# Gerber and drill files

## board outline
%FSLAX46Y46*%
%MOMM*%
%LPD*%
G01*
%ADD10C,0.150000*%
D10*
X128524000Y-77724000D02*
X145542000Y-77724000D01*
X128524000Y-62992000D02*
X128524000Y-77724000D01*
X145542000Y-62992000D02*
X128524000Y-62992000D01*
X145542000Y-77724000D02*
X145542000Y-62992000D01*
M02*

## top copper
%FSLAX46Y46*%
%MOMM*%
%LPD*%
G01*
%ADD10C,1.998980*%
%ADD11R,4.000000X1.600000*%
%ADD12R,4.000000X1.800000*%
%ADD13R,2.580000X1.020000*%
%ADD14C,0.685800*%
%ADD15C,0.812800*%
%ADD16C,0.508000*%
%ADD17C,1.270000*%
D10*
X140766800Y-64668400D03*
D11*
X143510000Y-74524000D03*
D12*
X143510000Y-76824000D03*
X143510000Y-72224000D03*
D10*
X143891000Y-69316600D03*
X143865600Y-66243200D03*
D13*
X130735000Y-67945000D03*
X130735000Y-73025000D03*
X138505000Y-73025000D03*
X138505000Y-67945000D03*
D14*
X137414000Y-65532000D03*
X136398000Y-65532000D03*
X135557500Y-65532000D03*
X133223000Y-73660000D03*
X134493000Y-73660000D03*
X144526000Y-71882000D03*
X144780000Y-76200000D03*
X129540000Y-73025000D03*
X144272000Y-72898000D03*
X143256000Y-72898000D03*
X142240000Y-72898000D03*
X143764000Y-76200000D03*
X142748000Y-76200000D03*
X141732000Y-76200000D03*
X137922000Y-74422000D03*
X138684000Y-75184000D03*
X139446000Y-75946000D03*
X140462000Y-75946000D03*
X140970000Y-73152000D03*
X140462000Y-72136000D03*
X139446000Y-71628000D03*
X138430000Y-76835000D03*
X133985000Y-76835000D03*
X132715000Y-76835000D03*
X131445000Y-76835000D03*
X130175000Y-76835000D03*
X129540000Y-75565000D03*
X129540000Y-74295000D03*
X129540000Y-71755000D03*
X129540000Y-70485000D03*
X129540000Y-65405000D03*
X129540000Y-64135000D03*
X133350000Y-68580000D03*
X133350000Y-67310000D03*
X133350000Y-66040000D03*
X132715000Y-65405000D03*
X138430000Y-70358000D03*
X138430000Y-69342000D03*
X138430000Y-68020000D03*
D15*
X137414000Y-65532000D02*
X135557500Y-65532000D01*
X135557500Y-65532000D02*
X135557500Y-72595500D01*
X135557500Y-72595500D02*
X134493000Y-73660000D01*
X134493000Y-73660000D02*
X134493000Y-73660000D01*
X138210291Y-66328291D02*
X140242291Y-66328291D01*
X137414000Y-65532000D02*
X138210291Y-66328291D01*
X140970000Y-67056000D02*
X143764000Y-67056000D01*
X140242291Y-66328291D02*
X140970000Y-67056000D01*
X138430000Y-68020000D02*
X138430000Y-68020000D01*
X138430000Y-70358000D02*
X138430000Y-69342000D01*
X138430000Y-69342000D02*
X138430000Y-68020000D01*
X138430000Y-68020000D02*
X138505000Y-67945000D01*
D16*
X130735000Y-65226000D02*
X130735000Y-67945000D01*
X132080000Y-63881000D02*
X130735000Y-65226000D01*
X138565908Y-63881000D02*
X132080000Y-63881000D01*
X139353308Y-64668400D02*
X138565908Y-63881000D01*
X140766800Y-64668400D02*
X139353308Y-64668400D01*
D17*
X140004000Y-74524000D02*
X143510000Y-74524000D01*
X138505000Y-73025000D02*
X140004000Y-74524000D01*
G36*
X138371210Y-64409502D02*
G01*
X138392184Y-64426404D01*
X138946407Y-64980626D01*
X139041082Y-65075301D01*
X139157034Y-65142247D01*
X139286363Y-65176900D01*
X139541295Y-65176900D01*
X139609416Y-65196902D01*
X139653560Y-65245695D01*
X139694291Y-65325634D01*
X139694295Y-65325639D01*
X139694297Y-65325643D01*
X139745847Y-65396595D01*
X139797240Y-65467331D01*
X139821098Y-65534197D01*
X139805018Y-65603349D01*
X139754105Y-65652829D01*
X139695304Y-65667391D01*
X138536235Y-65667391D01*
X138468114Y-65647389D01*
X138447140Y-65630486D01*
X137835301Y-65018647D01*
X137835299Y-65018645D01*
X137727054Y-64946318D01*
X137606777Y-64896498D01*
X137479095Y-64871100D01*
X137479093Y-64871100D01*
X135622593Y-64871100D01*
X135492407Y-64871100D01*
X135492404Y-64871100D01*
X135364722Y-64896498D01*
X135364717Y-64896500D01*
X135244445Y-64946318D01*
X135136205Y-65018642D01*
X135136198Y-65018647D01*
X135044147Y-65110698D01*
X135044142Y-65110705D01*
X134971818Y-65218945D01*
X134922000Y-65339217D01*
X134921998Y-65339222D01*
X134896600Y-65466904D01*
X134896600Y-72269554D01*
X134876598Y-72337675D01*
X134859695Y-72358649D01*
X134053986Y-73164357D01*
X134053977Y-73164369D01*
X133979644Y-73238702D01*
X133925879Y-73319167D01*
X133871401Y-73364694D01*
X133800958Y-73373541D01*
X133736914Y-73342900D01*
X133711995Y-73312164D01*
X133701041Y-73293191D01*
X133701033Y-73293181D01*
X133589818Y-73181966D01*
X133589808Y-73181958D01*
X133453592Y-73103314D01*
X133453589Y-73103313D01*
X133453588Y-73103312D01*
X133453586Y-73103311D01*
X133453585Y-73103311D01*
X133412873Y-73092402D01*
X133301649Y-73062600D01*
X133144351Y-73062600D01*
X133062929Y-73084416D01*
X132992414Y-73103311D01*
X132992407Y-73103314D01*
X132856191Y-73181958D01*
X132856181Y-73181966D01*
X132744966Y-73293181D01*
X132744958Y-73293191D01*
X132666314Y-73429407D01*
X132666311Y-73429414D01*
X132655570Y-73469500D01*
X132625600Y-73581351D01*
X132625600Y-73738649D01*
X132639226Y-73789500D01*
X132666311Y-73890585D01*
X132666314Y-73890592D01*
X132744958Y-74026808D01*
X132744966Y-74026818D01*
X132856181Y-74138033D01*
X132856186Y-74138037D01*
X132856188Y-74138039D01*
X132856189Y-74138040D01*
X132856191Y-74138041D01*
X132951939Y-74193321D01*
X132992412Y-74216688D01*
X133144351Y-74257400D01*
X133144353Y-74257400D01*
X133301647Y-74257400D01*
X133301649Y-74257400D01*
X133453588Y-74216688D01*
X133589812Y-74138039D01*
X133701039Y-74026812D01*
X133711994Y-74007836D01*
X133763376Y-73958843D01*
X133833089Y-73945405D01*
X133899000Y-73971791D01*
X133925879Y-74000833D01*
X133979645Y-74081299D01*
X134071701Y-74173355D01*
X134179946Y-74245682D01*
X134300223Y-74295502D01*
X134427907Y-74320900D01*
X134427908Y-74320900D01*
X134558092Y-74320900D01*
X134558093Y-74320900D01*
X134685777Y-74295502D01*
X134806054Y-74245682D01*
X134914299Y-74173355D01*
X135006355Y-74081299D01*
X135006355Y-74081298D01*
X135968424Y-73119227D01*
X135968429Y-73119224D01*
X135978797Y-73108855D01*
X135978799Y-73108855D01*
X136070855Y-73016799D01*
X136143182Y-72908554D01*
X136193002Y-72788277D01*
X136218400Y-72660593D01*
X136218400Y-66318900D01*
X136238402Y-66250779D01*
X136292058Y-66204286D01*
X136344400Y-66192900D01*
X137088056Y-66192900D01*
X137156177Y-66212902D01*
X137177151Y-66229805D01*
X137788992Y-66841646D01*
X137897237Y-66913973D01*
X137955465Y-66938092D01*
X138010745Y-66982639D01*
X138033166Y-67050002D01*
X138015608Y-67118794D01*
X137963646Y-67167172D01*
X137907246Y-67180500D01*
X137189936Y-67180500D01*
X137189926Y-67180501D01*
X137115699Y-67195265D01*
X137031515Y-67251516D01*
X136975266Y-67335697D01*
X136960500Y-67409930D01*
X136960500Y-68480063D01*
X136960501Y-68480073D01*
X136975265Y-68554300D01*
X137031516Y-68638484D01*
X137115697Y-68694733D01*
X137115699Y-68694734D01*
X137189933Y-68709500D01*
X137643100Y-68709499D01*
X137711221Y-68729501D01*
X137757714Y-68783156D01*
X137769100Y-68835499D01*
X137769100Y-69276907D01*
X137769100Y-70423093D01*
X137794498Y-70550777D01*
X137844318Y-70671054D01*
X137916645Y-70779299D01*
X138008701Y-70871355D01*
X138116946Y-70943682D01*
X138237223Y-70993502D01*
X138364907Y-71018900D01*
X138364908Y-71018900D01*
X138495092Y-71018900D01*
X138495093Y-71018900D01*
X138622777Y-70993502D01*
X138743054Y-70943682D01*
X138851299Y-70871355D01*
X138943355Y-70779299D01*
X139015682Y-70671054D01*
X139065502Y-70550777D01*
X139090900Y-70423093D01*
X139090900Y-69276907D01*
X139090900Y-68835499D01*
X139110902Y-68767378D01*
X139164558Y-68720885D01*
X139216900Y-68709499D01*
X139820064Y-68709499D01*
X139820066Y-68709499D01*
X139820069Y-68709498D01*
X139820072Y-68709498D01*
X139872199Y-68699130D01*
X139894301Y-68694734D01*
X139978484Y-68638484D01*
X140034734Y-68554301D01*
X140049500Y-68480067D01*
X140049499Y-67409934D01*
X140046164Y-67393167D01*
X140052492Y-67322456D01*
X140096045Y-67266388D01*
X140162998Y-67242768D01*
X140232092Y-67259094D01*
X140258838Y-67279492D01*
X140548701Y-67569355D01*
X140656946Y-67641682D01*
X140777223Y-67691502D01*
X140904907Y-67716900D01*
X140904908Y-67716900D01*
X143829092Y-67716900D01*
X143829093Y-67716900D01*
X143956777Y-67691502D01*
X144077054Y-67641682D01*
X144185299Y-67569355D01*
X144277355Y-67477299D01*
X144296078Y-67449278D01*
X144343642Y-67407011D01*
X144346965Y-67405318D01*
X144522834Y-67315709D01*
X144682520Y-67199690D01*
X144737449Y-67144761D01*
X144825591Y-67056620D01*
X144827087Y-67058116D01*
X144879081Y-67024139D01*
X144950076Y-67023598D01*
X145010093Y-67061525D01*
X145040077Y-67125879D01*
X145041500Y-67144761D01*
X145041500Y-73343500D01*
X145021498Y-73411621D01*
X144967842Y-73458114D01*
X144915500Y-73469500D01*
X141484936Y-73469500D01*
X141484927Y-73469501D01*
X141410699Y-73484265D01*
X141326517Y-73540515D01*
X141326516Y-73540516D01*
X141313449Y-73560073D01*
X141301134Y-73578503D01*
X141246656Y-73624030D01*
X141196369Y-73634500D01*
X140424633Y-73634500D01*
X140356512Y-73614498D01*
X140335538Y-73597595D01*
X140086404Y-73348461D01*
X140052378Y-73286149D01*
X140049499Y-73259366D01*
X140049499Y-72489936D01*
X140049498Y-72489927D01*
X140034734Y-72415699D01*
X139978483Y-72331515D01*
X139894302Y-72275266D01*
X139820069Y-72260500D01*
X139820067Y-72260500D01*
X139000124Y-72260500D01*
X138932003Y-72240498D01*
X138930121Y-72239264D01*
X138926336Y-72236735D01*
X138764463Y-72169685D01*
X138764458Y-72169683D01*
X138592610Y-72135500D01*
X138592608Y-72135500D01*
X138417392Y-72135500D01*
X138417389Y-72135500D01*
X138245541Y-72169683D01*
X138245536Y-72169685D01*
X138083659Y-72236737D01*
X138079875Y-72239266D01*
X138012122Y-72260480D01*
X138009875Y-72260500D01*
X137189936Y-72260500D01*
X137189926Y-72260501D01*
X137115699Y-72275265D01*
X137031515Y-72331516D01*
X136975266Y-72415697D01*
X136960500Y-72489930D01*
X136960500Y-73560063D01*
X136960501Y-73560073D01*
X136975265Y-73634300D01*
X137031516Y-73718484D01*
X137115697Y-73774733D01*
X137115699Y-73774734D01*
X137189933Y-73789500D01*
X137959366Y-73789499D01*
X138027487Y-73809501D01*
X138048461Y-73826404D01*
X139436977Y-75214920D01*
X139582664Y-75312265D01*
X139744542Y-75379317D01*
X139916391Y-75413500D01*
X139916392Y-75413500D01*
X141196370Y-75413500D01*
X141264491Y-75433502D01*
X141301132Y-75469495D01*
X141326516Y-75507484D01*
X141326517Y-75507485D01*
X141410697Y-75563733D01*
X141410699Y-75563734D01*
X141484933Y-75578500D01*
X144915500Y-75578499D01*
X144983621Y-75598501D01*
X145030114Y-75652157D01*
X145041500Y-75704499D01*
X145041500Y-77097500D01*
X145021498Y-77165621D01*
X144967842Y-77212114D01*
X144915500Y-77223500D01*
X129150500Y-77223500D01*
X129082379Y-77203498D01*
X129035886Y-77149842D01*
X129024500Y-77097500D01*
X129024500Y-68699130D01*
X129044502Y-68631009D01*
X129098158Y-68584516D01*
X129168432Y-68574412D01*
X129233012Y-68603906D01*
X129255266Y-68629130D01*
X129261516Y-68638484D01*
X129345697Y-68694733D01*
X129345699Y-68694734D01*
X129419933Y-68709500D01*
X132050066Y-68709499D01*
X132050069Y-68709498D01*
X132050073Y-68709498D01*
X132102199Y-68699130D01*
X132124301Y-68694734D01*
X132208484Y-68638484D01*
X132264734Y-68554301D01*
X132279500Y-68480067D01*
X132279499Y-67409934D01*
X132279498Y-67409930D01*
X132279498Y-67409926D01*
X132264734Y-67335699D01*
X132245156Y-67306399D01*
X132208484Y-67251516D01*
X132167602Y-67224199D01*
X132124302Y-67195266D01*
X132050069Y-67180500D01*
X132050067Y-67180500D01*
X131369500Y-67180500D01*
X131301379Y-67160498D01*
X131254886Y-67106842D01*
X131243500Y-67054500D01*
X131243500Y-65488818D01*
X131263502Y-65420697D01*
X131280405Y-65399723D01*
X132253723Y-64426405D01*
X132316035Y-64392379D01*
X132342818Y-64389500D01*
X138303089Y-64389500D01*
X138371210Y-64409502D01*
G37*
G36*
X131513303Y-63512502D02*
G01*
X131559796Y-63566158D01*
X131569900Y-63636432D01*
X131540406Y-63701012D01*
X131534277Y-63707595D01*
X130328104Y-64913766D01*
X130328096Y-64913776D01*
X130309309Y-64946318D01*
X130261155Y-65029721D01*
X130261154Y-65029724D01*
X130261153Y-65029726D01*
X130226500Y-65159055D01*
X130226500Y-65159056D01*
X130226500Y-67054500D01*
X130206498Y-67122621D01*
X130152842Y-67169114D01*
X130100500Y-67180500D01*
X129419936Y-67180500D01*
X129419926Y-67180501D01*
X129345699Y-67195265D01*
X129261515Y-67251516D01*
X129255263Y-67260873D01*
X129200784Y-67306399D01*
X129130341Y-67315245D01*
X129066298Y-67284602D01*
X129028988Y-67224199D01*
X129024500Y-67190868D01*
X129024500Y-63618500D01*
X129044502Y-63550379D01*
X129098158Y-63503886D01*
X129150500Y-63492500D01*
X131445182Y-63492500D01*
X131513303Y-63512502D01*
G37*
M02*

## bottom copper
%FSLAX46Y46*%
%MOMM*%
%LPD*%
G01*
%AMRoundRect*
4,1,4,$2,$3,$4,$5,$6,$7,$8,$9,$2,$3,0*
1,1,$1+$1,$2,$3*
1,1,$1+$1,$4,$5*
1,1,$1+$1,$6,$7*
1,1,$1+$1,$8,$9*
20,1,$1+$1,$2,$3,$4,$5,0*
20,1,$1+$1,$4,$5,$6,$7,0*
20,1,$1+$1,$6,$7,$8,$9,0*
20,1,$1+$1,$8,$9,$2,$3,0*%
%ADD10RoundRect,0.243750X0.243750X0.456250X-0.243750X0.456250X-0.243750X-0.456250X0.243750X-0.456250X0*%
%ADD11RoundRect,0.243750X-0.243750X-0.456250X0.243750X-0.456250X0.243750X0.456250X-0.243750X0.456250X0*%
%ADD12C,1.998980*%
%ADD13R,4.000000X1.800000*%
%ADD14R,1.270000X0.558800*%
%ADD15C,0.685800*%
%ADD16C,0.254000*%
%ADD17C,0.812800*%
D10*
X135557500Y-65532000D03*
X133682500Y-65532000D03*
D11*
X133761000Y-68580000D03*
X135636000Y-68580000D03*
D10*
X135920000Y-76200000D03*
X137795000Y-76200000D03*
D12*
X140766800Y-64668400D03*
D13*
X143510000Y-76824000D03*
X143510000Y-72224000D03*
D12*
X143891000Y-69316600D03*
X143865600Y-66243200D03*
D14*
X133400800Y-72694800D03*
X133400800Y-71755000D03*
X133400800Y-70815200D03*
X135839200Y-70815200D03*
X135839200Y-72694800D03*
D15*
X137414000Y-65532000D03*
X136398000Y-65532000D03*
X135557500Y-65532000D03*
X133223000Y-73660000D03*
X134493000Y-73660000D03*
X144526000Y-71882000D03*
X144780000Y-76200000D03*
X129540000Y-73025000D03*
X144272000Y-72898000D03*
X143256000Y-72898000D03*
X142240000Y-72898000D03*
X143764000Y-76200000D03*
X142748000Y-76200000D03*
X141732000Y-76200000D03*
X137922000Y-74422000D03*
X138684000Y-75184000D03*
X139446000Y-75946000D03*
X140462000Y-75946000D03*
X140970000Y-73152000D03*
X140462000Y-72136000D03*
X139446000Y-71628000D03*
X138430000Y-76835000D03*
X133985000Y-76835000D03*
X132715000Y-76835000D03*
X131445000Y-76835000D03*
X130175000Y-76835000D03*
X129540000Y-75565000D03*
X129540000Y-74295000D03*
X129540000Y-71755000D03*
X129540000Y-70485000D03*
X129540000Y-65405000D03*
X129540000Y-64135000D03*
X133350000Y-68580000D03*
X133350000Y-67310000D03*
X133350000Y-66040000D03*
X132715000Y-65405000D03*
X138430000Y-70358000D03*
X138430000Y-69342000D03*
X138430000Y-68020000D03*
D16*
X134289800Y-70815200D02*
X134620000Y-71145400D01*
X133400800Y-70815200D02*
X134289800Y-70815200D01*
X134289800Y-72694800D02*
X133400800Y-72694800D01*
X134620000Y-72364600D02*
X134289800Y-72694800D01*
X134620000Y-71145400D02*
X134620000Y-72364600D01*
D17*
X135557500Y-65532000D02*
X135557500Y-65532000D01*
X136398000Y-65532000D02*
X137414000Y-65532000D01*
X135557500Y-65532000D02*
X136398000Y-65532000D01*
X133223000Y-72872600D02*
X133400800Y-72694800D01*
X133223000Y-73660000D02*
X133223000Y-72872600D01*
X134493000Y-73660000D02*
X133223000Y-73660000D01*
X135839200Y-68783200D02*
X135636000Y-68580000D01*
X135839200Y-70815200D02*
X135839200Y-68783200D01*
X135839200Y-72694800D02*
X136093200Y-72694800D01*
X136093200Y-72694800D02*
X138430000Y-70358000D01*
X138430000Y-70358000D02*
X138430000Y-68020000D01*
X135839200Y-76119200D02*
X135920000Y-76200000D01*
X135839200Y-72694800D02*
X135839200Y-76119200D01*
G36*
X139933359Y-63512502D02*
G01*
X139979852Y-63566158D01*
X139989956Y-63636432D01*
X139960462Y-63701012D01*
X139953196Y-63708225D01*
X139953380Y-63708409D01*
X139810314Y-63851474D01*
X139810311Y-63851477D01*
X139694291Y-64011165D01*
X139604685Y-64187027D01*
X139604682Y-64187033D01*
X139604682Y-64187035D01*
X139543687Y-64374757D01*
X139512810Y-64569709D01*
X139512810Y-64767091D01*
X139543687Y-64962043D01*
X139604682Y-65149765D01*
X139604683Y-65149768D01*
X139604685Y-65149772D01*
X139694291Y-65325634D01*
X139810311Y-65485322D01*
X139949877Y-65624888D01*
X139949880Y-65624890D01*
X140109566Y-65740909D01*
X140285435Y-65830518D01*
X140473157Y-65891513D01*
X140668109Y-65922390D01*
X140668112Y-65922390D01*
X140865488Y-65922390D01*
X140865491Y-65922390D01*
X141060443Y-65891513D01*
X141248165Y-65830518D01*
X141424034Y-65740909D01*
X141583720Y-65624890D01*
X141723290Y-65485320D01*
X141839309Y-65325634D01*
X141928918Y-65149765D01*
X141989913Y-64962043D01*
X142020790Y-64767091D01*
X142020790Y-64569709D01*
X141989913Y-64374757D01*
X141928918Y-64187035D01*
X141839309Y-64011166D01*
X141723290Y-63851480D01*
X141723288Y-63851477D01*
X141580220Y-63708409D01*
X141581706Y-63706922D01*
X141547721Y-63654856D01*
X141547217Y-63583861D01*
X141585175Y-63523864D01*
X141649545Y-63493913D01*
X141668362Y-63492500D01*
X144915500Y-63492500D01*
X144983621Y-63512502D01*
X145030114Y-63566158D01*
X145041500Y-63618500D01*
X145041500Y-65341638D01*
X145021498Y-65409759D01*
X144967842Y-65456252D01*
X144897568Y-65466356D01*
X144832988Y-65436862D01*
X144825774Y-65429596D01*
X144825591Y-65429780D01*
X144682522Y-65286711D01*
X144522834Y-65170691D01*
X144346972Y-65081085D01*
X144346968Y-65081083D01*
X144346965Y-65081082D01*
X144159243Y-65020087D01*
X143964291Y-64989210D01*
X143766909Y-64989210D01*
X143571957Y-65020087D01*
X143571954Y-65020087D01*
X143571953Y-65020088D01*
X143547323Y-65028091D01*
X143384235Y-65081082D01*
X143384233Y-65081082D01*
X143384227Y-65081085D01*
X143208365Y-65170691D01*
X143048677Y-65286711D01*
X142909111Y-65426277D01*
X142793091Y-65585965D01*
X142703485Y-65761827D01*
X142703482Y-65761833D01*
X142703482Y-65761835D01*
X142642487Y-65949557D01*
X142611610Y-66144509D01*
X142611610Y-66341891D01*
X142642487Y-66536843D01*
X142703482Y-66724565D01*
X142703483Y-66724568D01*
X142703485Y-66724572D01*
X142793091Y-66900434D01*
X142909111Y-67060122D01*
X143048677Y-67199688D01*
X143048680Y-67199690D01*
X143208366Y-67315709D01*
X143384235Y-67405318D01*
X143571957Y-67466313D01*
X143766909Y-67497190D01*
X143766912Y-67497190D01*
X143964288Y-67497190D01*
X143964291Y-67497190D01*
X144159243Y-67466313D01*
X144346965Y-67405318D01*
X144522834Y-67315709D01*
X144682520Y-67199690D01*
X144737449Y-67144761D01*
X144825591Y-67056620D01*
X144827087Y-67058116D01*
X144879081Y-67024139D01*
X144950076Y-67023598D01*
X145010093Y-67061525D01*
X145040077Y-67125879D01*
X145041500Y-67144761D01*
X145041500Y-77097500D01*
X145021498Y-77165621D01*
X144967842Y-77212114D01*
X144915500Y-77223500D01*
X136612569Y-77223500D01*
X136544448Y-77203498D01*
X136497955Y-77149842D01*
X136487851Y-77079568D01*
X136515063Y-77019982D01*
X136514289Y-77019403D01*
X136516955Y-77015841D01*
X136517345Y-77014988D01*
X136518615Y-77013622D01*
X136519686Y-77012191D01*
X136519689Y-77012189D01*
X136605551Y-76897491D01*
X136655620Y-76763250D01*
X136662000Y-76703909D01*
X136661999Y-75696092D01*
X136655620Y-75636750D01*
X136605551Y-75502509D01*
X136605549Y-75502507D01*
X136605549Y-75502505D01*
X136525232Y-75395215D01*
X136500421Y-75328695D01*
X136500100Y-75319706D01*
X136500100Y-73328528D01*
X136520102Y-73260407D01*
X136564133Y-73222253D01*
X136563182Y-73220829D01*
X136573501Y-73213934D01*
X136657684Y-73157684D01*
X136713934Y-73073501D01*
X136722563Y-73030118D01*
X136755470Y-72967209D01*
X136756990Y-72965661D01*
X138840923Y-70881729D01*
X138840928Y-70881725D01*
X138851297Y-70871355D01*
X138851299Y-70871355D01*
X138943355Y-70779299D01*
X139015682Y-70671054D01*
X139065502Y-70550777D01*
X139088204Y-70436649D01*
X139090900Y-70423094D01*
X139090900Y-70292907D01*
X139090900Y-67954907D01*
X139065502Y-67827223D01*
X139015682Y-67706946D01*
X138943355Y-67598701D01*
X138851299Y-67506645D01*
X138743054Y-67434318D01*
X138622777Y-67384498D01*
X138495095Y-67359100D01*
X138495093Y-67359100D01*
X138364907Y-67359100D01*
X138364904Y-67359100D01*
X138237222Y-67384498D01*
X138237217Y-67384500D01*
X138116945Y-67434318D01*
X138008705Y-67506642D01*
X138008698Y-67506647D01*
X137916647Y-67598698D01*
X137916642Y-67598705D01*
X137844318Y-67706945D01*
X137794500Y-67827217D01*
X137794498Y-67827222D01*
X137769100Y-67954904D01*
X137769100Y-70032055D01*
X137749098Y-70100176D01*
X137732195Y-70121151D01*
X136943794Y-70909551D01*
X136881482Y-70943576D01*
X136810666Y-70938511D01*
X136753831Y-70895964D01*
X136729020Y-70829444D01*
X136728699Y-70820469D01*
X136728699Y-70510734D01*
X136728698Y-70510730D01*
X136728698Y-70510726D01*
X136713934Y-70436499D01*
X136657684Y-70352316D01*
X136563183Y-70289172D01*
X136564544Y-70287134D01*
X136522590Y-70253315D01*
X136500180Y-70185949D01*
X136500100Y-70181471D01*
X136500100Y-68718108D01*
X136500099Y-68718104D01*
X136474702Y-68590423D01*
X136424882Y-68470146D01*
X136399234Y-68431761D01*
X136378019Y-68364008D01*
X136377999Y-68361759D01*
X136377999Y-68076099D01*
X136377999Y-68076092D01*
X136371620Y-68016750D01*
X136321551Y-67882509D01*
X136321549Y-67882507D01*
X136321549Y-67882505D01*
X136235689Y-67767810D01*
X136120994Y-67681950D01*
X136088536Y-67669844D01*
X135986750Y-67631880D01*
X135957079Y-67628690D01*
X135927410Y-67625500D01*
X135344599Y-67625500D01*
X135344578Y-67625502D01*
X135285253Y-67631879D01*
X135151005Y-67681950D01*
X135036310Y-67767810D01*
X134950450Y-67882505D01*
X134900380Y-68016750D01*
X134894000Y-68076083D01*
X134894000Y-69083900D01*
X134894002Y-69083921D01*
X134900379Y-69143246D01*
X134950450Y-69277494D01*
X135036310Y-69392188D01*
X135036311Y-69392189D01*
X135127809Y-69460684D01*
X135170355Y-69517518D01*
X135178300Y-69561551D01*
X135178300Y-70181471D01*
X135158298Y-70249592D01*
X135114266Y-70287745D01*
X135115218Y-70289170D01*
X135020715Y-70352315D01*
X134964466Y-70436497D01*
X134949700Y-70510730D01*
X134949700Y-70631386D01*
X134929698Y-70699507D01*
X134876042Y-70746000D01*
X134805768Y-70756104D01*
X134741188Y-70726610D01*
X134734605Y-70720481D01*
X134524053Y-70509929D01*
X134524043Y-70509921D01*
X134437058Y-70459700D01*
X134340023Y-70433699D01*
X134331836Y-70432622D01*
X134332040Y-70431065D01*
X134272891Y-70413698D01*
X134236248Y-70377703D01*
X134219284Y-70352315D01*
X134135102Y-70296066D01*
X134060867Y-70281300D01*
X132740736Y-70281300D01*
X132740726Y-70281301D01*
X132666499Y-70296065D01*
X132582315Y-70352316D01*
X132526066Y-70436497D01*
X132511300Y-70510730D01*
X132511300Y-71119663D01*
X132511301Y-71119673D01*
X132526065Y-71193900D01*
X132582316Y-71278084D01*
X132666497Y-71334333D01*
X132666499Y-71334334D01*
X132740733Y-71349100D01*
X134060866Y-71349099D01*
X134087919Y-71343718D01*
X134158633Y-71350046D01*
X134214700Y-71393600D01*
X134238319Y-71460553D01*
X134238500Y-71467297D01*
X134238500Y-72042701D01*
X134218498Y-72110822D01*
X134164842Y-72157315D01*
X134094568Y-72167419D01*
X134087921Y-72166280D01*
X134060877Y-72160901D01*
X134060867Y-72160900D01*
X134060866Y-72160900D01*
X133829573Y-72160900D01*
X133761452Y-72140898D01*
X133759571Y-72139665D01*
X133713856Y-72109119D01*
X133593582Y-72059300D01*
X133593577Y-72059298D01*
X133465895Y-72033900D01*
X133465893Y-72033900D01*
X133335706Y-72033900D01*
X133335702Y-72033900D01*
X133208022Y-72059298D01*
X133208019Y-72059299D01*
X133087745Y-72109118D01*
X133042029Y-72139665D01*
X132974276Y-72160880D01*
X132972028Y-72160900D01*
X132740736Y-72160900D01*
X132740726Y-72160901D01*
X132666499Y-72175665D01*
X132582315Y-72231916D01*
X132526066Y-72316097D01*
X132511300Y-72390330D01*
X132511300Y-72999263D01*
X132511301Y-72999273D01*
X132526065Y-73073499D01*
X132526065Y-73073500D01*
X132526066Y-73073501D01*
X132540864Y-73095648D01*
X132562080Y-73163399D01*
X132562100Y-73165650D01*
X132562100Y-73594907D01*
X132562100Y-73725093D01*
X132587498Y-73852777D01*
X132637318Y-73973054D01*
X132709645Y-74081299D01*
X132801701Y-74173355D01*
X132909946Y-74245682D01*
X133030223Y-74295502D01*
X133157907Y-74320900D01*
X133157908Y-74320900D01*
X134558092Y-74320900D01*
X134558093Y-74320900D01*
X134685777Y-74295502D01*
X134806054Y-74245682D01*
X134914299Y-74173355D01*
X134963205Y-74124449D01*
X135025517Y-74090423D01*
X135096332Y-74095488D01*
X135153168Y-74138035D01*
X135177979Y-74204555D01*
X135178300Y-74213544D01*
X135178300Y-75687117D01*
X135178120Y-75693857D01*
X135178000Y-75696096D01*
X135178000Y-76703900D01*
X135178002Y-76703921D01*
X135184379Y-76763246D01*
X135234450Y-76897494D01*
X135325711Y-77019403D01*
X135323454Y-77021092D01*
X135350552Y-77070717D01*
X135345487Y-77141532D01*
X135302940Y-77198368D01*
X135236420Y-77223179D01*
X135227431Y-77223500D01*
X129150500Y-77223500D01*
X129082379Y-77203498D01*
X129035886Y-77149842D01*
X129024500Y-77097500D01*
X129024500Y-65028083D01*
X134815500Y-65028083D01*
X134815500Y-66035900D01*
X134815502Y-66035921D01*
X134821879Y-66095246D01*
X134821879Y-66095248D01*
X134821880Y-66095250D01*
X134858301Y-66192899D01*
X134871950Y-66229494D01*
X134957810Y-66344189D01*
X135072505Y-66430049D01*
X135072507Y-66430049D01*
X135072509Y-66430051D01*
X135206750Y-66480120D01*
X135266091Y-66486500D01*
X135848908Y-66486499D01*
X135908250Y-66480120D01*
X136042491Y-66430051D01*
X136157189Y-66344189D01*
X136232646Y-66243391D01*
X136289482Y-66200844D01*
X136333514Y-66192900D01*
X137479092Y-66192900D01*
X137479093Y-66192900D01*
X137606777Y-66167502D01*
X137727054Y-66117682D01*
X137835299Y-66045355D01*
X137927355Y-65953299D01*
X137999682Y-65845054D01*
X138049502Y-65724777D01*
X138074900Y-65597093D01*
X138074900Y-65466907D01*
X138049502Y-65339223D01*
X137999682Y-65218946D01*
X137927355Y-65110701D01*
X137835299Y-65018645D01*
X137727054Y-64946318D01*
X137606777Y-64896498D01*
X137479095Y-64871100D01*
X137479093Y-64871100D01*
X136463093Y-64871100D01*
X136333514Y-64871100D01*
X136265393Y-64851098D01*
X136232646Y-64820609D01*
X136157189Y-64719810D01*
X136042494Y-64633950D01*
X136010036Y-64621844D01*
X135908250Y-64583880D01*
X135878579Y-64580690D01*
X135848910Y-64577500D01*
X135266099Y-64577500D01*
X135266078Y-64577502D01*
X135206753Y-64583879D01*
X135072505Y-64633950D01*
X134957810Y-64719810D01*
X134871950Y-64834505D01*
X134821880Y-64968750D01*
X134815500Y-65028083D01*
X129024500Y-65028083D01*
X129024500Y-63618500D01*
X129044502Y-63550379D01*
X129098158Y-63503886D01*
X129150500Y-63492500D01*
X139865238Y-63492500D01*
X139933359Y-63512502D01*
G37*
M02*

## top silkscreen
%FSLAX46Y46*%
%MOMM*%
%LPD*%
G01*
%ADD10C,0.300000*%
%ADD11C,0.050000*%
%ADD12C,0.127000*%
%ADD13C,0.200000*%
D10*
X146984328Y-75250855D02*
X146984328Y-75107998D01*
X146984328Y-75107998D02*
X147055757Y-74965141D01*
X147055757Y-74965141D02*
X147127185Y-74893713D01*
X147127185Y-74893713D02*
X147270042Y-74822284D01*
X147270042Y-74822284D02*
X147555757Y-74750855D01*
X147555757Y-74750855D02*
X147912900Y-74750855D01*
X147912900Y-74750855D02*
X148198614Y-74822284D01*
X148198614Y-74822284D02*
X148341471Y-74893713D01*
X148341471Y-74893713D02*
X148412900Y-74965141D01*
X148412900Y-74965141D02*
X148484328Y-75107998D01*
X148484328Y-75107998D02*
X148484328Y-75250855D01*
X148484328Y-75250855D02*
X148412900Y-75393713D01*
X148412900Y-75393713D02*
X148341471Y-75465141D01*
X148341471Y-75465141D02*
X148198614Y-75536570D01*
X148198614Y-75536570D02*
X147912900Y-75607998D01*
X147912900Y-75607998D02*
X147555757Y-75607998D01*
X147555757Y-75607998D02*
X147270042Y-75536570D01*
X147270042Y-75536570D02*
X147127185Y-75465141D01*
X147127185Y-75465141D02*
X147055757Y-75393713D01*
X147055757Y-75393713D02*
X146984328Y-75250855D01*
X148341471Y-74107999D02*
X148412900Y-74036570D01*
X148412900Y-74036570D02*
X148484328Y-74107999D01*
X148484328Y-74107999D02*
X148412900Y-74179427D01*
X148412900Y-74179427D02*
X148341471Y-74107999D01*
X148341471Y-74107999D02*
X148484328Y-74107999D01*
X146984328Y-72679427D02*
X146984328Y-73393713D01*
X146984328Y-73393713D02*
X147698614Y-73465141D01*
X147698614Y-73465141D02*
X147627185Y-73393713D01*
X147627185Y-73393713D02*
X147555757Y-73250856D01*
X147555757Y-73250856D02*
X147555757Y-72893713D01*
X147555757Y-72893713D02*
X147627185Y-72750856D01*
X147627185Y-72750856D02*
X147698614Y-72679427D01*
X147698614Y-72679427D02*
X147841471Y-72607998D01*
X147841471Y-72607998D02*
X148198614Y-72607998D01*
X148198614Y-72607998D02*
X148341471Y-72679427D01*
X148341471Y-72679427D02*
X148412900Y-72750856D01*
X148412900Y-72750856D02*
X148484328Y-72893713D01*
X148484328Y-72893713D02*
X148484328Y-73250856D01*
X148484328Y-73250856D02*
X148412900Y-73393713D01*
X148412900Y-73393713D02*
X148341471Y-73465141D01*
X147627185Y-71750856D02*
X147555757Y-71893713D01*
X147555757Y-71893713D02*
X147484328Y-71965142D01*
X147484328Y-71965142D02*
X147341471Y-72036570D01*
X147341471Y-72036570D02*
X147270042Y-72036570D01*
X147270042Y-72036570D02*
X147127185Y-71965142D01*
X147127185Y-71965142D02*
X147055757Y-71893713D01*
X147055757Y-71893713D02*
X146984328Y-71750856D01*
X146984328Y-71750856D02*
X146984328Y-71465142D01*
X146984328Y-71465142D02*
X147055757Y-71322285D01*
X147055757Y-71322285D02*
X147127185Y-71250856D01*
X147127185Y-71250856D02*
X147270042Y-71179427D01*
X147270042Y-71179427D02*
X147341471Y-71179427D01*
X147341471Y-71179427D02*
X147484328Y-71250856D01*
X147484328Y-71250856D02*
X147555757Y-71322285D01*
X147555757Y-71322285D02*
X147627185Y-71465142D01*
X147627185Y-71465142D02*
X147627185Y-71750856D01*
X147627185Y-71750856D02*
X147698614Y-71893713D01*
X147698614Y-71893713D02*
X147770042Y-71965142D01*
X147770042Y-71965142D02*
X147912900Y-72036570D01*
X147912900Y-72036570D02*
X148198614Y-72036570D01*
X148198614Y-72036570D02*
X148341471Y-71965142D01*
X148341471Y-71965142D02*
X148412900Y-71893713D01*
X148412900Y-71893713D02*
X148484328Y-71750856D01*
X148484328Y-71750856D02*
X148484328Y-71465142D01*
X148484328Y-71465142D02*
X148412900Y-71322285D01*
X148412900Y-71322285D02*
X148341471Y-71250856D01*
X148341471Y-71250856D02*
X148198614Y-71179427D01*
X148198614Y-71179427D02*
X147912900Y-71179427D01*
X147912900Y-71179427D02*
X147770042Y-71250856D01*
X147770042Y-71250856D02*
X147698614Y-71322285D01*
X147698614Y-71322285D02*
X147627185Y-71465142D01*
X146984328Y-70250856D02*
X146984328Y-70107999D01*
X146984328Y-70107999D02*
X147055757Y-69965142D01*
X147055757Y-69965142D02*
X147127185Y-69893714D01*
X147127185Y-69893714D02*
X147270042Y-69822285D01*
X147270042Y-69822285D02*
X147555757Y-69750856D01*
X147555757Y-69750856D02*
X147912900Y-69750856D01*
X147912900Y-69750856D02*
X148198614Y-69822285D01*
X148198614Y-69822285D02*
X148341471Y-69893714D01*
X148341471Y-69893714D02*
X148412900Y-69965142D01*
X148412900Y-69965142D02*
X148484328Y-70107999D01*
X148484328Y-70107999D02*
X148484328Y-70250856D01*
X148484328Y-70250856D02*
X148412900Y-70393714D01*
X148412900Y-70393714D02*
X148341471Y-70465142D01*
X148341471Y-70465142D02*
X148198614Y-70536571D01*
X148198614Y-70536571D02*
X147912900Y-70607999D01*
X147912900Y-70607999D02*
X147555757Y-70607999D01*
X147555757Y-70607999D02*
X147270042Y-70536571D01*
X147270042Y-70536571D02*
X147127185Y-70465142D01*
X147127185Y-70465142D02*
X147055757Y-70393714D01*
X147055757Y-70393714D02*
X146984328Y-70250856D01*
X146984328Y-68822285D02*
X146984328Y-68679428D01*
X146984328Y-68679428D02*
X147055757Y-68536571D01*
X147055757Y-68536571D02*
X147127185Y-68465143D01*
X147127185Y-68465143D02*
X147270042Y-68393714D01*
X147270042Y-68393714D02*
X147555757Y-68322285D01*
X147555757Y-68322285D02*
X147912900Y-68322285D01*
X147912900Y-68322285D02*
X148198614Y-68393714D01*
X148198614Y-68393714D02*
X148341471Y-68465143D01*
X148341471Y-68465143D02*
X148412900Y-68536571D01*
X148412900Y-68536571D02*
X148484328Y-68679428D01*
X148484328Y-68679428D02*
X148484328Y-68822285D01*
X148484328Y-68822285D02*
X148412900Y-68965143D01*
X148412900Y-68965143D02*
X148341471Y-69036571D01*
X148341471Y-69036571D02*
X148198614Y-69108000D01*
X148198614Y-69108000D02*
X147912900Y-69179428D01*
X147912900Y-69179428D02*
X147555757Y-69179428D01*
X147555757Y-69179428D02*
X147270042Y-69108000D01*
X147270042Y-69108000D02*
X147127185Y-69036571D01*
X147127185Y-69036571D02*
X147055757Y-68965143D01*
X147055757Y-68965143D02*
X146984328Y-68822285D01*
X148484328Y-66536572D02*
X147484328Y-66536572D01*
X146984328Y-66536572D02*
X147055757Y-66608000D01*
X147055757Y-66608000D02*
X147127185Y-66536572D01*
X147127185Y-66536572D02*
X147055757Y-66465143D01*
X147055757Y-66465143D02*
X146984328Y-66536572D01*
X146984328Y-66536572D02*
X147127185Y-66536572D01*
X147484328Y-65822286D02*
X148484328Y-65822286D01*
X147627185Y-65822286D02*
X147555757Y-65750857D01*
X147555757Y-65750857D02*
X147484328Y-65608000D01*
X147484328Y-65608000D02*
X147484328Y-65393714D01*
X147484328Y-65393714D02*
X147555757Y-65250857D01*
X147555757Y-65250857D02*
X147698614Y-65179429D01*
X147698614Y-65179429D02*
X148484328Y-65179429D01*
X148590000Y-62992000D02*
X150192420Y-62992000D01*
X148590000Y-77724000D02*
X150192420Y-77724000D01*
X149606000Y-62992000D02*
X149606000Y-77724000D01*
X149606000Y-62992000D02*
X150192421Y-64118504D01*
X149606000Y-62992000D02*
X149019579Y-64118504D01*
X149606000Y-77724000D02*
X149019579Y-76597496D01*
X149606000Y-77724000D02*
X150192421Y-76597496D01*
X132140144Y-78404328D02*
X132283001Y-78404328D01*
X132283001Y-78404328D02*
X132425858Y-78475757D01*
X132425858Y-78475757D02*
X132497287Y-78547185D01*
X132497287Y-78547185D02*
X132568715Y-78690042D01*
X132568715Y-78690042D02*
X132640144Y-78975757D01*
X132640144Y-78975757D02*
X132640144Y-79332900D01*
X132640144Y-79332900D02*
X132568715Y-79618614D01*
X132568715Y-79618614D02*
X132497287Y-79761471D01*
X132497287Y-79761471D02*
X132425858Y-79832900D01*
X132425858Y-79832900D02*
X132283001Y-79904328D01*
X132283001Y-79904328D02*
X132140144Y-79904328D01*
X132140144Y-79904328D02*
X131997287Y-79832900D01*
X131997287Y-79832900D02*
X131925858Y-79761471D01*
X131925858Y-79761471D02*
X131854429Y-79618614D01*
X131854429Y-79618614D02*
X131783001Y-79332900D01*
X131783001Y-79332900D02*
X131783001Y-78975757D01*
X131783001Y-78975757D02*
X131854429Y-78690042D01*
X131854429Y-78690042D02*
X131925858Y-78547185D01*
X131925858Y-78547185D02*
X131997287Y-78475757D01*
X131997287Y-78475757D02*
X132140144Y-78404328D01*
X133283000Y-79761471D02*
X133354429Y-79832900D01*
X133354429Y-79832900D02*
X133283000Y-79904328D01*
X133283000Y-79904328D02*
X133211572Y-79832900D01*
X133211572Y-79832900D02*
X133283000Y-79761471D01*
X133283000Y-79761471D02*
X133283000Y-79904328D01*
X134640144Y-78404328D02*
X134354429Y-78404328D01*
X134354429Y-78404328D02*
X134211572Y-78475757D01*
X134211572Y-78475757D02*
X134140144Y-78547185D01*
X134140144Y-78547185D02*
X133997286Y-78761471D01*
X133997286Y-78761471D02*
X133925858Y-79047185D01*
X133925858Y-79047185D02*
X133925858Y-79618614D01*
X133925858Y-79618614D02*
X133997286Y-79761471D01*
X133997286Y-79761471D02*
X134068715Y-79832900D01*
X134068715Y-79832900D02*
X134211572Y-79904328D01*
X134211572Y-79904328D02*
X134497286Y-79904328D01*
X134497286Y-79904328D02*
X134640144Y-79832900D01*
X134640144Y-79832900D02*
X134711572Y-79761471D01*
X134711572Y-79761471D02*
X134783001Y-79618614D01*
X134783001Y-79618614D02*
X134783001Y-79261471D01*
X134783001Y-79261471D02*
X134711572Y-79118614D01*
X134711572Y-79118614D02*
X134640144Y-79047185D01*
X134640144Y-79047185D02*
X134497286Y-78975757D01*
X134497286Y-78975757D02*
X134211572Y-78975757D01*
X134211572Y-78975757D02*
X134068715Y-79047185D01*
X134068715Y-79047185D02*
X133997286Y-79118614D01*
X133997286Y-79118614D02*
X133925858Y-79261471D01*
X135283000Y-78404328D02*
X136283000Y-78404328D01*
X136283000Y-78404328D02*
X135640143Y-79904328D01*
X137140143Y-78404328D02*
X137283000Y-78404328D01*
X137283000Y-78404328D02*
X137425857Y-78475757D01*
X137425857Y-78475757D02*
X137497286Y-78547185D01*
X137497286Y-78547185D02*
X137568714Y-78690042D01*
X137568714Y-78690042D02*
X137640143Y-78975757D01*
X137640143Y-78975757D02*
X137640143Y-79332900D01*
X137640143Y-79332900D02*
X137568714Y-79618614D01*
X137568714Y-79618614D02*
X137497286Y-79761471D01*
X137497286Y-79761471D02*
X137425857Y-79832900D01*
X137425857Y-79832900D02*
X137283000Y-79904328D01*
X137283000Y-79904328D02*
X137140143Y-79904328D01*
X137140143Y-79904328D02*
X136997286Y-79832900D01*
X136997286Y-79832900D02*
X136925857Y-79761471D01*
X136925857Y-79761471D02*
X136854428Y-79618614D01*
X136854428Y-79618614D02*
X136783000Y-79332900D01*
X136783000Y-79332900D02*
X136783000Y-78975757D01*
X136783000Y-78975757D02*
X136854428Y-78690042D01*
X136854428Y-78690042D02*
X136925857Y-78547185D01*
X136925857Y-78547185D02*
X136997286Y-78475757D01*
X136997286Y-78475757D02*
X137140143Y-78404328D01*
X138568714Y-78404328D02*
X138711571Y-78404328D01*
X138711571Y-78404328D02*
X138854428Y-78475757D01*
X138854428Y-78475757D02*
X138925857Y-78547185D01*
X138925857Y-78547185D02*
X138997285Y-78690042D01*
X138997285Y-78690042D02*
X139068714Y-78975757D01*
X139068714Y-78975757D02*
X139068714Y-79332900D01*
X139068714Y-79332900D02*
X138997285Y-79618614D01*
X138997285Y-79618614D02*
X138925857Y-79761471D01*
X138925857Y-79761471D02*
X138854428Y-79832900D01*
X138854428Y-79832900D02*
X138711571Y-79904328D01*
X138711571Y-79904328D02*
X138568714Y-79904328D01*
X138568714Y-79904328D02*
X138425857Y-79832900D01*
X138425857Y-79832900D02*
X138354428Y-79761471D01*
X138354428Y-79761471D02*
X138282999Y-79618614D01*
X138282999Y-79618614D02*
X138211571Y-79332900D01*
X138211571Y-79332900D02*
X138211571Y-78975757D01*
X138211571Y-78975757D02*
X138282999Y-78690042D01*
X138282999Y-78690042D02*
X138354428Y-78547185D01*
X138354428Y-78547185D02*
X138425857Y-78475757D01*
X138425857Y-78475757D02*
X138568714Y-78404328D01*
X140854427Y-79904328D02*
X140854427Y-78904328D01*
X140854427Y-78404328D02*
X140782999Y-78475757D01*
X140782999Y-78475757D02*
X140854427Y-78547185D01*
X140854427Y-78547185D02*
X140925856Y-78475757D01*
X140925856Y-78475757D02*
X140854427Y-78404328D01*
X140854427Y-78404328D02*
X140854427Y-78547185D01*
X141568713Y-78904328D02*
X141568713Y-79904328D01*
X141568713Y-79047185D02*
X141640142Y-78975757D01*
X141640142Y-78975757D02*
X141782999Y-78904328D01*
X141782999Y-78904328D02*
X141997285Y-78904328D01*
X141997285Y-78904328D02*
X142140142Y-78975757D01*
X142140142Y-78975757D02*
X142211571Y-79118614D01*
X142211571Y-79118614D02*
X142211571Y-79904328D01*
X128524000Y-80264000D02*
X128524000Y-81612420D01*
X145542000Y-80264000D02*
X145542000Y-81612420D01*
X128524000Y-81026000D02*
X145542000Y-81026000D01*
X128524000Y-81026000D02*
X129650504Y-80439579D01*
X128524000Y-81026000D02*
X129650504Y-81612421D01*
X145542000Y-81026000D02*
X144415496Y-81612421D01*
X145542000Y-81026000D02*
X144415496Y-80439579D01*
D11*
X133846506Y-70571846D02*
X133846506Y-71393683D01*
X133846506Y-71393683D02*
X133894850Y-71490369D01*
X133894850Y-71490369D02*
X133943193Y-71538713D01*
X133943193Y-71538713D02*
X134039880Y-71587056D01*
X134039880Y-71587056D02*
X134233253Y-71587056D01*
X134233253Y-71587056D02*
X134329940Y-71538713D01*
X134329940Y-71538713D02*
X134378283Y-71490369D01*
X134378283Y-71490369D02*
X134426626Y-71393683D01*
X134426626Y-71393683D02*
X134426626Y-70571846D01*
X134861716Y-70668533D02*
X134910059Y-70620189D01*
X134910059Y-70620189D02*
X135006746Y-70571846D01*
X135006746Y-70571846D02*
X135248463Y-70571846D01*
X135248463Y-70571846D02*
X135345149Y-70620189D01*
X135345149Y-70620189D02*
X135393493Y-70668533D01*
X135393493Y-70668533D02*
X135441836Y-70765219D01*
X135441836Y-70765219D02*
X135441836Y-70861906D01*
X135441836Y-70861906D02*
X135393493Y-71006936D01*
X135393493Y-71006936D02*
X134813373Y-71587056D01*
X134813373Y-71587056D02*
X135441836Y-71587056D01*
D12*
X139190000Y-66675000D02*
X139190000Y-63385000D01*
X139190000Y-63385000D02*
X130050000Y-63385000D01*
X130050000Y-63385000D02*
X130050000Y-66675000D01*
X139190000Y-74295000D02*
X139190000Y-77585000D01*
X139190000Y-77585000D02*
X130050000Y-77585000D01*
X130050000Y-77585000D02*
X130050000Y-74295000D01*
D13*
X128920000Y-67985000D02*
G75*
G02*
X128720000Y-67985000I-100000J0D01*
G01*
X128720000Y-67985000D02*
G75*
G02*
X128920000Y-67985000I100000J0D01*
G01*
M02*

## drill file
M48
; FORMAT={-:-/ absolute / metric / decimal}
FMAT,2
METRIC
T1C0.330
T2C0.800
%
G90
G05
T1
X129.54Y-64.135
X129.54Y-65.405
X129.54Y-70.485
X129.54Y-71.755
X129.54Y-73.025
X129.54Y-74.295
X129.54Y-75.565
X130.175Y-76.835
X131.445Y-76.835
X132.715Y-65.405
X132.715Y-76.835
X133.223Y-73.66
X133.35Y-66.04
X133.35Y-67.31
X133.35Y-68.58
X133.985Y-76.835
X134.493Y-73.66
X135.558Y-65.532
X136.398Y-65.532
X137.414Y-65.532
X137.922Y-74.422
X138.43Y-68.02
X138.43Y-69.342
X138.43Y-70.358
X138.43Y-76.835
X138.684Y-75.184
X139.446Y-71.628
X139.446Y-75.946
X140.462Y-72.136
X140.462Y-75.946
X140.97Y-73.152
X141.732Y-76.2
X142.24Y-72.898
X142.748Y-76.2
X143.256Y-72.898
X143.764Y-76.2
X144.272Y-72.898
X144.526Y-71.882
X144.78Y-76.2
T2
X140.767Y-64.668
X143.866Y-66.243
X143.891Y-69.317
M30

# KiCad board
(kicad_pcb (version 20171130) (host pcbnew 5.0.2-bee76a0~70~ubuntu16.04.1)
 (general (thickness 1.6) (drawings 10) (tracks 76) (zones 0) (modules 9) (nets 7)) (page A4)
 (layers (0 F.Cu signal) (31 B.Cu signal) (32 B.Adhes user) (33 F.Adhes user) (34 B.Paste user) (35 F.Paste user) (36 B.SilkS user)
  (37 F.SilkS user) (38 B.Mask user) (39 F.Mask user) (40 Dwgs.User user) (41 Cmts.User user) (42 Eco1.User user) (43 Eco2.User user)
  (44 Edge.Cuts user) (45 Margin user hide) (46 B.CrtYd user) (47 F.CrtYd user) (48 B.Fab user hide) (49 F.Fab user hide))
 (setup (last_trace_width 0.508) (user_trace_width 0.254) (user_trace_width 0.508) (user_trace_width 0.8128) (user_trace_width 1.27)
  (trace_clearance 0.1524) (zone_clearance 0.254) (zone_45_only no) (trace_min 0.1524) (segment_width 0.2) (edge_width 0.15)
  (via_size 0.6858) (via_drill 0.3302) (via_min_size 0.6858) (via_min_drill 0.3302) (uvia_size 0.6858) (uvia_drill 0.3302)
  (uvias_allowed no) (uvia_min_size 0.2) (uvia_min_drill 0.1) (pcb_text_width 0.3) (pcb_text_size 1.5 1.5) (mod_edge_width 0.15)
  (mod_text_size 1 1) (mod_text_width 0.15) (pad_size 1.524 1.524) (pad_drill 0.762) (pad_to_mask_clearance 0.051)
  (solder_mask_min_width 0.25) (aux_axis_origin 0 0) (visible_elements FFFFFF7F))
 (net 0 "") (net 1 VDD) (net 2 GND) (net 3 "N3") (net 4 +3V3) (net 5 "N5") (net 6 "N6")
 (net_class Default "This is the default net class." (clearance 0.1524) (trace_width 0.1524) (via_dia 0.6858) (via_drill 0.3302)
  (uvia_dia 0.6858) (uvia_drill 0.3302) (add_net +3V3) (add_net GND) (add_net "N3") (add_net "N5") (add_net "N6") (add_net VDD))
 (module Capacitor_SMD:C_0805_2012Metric (layer B.Cu) (at 134.62 65.532 180)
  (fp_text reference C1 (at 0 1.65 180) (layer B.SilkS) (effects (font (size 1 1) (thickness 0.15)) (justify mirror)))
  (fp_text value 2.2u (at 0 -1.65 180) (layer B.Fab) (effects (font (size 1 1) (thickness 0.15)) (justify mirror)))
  (pad 1 smd roundrect (at -0.9375 0 180) (size 0.975 1.4) (layers B.Cu B.Paste B.Mask) (roundrect_rratio 0.25) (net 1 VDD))
  (pad 2 smd roundrect (at 0.9375 0 180) (size 0.975 1.4) (layers B.Cu B.Paste B.Mask) (roundrect_rratio 0.25) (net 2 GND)))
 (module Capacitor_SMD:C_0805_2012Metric (layer B.Cu) (at 134.6985 68.58)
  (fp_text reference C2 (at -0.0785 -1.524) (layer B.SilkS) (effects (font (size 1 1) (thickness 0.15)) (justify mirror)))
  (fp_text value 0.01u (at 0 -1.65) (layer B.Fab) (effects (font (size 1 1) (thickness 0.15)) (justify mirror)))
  (pad 1 smd roundrect (at -0.9375 0) (size 0.975 1.4) (layers B.Cu B.Paste B.Mask) (roundrect_rratio 0.25) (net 2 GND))
  (pad 2 smd roundrect (at 0.9375 0) (size 0.975 1.4) (layers B.Cu B.Paste B.Mask) (roundrect_rratio 0.25) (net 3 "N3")))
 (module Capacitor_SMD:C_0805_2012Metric (layer B.Cu) (at 136.8575 76.2 180)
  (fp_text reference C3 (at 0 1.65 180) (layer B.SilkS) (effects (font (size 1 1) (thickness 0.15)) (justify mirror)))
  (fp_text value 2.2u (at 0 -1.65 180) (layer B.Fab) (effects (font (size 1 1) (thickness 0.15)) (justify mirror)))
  (pad 2 smd roundrect (at 0.9375 0 180) (size 0.975 1.4) (layers B.Cu B.Paste B.Mask) (roundrect_rratio 0.25) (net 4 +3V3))
  (pad 1 smd roundrect (at -0.9375 0 180) (size 0.975 1.4) (layers B.Cu B.Paste B.Mask) (roundrect_rratio 0.25) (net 2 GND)))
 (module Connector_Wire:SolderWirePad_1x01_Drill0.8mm (layer F.Cu) (at 140.7668 64.6684)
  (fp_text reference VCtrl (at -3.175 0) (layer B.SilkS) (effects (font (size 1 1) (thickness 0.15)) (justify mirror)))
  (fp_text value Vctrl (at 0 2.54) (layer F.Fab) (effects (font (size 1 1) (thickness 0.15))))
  (pad 1 thru_hole circle (at 0 0) (size 1.99898 1.99898) (drill 0.8001) (layers *.Cu *.Mask) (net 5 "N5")))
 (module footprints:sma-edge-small (layer F.Cu) (at 143.51 74.524)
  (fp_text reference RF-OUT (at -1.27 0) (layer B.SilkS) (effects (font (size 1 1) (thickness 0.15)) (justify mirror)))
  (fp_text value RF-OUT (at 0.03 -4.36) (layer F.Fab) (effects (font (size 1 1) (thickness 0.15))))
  (pad 1 smd rect (at 0 0) (size 4 1.6) (layers F.Cu F.Mask) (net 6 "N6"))
  (pad 2 smd rect (at 0 3.2) (size 4 1.8) (drill (offset 0 -0.9)) (layers F.Cu F.Mask) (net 2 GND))
  (pad 2 smd rect (at 0 3.2) (size 4 1.8) (drill (offset 0 -0.9)) (layers B.Cu B.Mask) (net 2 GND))
  (pad 2 smd rect (at 0 -3.2) (size 4 1.8) (drill (offset 0 0.9)) (layers F.Cu F.Mask) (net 2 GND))
  (pad 2 smd rect (at 0 -3.2) (size 4 1.8) (drill (offset 0 0.9)) (layers B.Cu B.Mask) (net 2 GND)))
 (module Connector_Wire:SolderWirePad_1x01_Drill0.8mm (layer F.Cu) (at 143.891 69.3166)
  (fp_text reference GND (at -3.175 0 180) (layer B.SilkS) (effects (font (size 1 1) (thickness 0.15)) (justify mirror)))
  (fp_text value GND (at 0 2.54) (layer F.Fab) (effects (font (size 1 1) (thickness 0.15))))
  (pad 1 thru_hole circle (at 0 0) (size 1.99898 1.99898) (drill 0.8001) (layers *.Cu *.Mask) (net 2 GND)))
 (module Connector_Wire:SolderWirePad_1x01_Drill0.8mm (layer F.Cu) (at 143.8656 66.2432)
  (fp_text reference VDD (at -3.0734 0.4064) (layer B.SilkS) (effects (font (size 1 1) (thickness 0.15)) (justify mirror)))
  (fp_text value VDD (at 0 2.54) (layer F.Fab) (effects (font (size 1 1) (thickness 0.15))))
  (pad 1 thru_hole circle (at 0 0) (size 1.99898 1.99898) (drill 0.8001) (layers *.Cu *.Mask) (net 1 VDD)))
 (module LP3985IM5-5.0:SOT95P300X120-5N (layer B.Cu) (at 134.62 71.755)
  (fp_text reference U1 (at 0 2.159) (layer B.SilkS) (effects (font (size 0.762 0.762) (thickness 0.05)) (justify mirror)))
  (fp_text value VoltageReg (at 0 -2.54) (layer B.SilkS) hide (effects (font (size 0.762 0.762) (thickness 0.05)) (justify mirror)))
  (pad 1 smd rect (at -1.2192 0.9398) (size 1.27 0.5588) (layers B.Cu B.Paste B.Mask) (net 1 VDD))
  (pad 2 smd rect (at -1.2192 0) (size 1.27 0.5588) (layers B.Cu B.Paste B.Mask) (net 2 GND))
  (pad 3 smd rect (at -1.2192 -0.9398) (size 1.27 0.5588) (layers B.Cu B.Paste B.Mask) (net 1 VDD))
  (pad 4 smd rect (at 1.2192 -0.9398) (size 1.27 0.5588) (layers B.Cu B.Paste B.Mask) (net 3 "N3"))
  (pad 5 smd rect (at 1.2192 0.9398) (size 1.27 0.5588) (layers B.Cu B.Paste B.Mask) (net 4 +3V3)))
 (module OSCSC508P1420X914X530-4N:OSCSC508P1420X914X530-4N (layer F.Cu) (at 134.62 70.485 270)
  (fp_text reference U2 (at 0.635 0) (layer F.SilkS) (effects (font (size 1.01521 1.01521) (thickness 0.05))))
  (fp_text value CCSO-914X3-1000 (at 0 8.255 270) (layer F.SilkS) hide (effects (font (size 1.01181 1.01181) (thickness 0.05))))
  (fp_line (start -3.81 -4.57) (end -7.1 -4.57) (layer F.SilkS) (width 0.127))
  (fp_line (start -7.1 -4.57) (end -7.1 4.57) (layer F.SilkS) (width 0.127))
  (fp_line (start -7.1 4.57) (end -3.81 4.57) (layer F.SilkS) (width 0.127))
  (fp_line (start 3.81 -4.57) (end 7.1 -4.57) (layer F.SilkS) (width 0.127))
  (fp_line (start 7.1 -4.57) (end 7.1 4.57) (layer F.SilkS) (width 0.127))
  (fp_line (start 7.1 4.57) (end 3.81 4.57) (layer F.SilkS) (width 0.127))
  (fp_circle (center -2.5 5.8) (end -2.4 5.8) (layer F.SilkS) (width 0.2))
  (pad 1 smd rect (at -2.54 3.885 180) (size 2.58 1.02) (layers F.Cu F.Paste F.Mask) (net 5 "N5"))
  (pad 2 smd rect (at 2.54 3.885 180) (size 2.58 1.02) (layers F.Cu F.Paste F.Mask) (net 2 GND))
  (pad 3 smd rect (at 2.54 -3.885 180) (size 2.58 1.02) (layers F.Cu F.Paste F.Mask) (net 6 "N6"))
  (pad 4 smd rect (at -2.54 -3.885 180) (size 2.58 1.02) (layers F.Cu F.Paste F.Mask) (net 4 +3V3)))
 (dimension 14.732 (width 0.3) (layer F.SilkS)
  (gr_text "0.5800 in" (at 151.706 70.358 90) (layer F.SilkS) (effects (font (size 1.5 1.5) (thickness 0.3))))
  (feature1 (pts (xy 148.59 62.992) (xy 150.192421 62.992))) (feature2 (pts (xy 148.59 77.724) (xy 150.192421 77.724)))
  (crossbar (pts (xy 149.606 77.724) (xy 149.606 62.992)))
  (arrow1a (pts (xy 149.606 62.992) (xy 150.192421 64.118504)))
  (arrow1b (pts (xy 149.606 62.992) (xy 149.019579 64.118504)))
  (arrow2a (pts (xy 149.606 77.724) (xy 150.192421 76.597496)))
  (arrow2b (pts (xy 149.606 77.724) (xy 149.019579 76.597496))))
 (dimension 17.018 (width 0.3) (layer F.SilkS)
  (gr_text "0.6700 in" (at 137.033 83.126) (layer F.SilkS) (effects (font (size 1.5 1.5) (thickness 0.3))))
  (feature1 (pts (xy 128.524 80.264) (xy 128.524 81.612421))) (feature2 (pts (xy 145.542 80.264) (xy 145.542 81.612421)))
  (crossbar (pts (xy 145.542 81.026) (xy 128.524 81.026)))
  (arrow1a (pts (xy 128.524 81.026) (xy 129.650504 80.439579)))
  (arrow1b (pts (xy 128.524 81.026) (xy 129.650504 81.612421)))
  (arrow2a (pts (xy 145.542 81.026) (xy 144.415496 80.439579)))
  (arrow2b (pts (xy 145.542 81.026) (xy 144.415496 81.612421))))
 (gr_line (start 128.524 77.724) (end 145.542 77.724) (layer Edge.Cuts) (width 0.15))
 (gr_line (start 128.524 62.992) (end 128.524 77.724) (layer Edge.Cuts) (width 0.15))
 (gr_line (start 145.542 62.992) (end 128.524 62.992) (layer Edge.Cuts) (width 0.15))
 (gr_line (start 145.542 77.724) (end 145.542 62.992) (layer Edge.Cuts) (width 0.15))
 (segment (start 134.2898 70.8152) (end 134.62 71.1454) (width 0.254) (layer B.Cu) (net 1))
 (segment (start 133.4008 70.8152) (end 134.2898 70.8152) (width 0.254) (layer B.Cu) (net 1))
 (segment (start 134.2898 72.6948) (end 133.4008 72.6948) (width 0.254) (layer B.Cu) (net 1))
 (segment (start 134.62 72.3646) (end 134.2898 72.6948) (width 0.254) (layer B.Cu) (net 1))
 (segment (start 134.62 71.1454) (end 134.62 72.3646) (width 0.254) (layer B.Cu) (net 1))
 (via (at 137.414 65.532) (size 0.6858) (drill 0.3302) (layers F.Cu B.Cu) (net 1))
 (segment (start 135.5575 65.532) (end 135.5575 65.532) (width 0.8128) (layer B.Cu) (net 1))
 (segment (start 136.398 65.532) (end 137.414 65.532) (width 0.8128) (layer B.Cu) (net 1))
 (via (at 136.398 65.532) (size 0.6858) (drill 0.3302) (layers F.Cu B.Cu) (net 1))
 (segment (start 135.5575 65.532) (end 136.398 65.532) (width 0.8128) (layer B.Cu) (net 1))
 (via (at 135.5575 65.532) (size 0.6858) (drill 0.3302) (layers F.Cu B.Cu) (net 1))
 (segment (start 137.414 65.532) (end 135.5575 65.532) (width 0.8128) (layer F.Cu) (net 1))
 (segment (start 135.5575 65.532) (end 135.5575 72.5955) (width 0.8128) (layer F.Cu) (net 1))
 (via (at 133.223 73.66) (size 0.6858) (drill 0.3302) (layers F.Cu B.Cu) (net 1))
 (segment (start 135.5575 72.5955) (end 134.493 73.66) (width 0.8128) (layer F.Cu) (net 1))
 (segment (start 133.223 72.8726) (end 133.4008 72.6948) (width 0.8128) (layer B.Cu) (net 1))
 (segment (start 133.223 73.66) (end 133.223 72.8726) (width 0.8128) (layer B.Cu) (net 1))
 (segment (start 134.493 73.66) (end 134.493 73.66) (width 0.8128) (layer F.Cu) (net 1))
 (via (at 134.493 73.66) (size 0.6858) (drill 0.3302) (layers F.Cu B.Cu) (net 1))
 (segment (start 134.493 73.66) (end 133.223 73.66) (width 0.8128) (layer B.Cu) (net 1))
 (segment (start 138.210291 66.328291) (end 140.242291 66.328291) (width 0.8128) (layer F.Cu) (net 1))
 (segment (start 137.414 65.532) (end 138.210291 66.328291) (width 0.8128) (layer F.Cu) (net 1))
 (segment (start 140.97 67.056) (end 143.764 67.056) (width 0.8128) (layer F.Cu) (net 1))
 (segment (start 140.242291 66.328291) (end 140.97 67.056) (width 0.8128) (layer F.Cu) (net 1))
 (via (at 144.526 71.882) (size 0.6858) (drill 0.3302) (layers F.Cu B.Cu) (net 2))
 (via (at 144.78 76.2) (size 0.6858) (drill 0.3302) (layers F.Cu B.Cu) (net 2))
 (via (at 129.54 73.025) (size 0.6858) (drill 0.3302) (layers F.Cu B.Cu) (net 2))
 (via (at 144.272 72.898) (size 0.6858) (drill 0.3302) (layers F.Cu B.Cu) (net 2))
 (via (at 143.256 72.898) (size 0.6858) (drill 0.3302) (layers F.Cu B.Cu) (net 2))
 (via (at 142.24 72.898) (size 0.6858) (drill 0.3302) (layers F.Cu B.Cu) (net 2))
 (via (at 143.764 76.2) (size 0.6858) (drill 0.3302) (layers F.Cu B.Cu) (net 2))
 (via (at 142.748 76.2) (size 0.6858) (drill 0.3302) (layers F.Cu B.Cu) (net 2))
 (via (at 141.732 76.2) (size 0.6858) (drill 0.3302) (layers F.Cu B.Cu) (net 2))
 (via (at 137.922 74.422) (size 0.6858) (drill 0.3302) (layers F.Cu B.Cu) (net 2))
 (via (at 138.684 75.184) (size 0.6858) (drill 0.3302) (layers F.Cu B.Cu) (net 2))
 (via (at 139.446 75.946) (size 0.6858) (drill 0.3302) (layers F.Cu B.Cu) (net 2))
 (via (at 140.462 75.946) (size 0.6858) (drill 0.3302) (layers F.Cu B.Cu) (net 2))
 (via (at 140.97 73.152) (size 0.6858) (drill 0.3302) (layers F.Cu B.Cu) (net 2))
 (via (at 140.462 72.136) (size 0.6858) (drill 0.3302) (layers F.Cu B.Cu) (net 2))
 (via (at 139.446 71.628) (size 0.6858) (drill 0.3302) (layers F.Cu B.Cu) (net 2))
 (via (at 138.43 76.835) (size 0.6858) (drill 0.3302) (layers F.Cu B.Cu) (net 2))
 (via (at 133.985 76.835) (size 0.6858) (drill 0.3302) (layers F.Cu B.Cu) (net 2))
 (via (at 132.715 76.835) (size 0.6858) (drill 0.3302) (layers F.Cu B.Cu) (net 2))
 (via (at 131.445 76.835) (size 0.6858) (drill 0.3302) (layers F.Cu B.Cu) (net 2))
 (via (at 130.175 76.835) (size 0.6858) (drill 0.3302) (layers F.Cu B.Cu) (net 2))
 (via (at 129.54 75.565) (size 0.6858) (drill 0.3302) (layers F.Cu B.Cu) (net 2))
 (via (at 129.54 74.295) (size 0.6858) (drill 0.3302) (layers F.Cu B.Cu) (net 2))
 (via (at 129.54 71.755) (size 0.6858) (drill 0.3302) (layers F.Cu B.Cu) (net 2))
 (via (at 129.54 70.485) (size 0.6858) (drill 0.3302) (layers F.Cu B.Cu) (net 2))
 (via (at 129.54 65.405) (size 0.6858) (drill 0.3302) (layers F.Cu B.Cu) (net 2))
 (via (at 129.54 64.135) (size 0.6858) (drill 0.3302) (layers F.Cu B.Cu) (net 2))
 (via (at 133.35 68.58) (size 0.6858) (drill 0.3302) (layers F.Cu B.Cu) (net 2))
 (via (at 133.35 67.31) (size 0.6858) (drill 0.3302) (layers F.Cu B.Cu) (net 2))
 (via (at 133.35 66.04) (size 0.6858) (drill 0.3302) (layers F.Cu B.Cu) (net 2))
 (via (at 132.715 65.405) (size 0.6858) (drill 0.3302) (layers F.Cu B.Cu) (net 2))
 (segment (start 135.8392 68.7832) (end 135.636 68.58) (width 0.8128) (layer B.Cu) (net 3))
 (segment (start 135.8392 70.8152) (end 135.8392 68.7832) (width 0.8128) (layer B.Cu) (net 3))
 (via (at 138.43 70.358) (size 0.6858) (drill 0.3302) (layers F.Cu B.Cu) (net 4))
 (segment (start 135.8392 72.6948) (end 136.0932 72.6948) (width 0.8128) (layer B.Cu) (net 4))
 (segment (start 136.0932 72.6948) (end 138.43 70.358) (width 0.8128) (layer B.Cu) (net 4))
 (segment (start 138.43 68.02) (end 138.43 68.02) (width 0.8128) (layer F.Cu) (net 4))
 (segment (start 138.43 70.358) (end 138.43 69.342) (width 0.8128) (layer F.Cu) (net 4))
 (segment (start 138.43 69.342) (end 138.43 68.02) (width 0.8128) (layer F.Cu) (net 4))
 (via (at 138.43 69.342) (size 0.6858) (drill 0.3302) (layers F.Cu B.Cu) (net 4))
 (segment (start 138.43 68.02) (end 138.505 67.945) (width 0.8128) (layer F.Cu) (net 4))
 (via (at 138.43 68.02) (size 0.6858) (drill 0.3302) (layers F.Cu B.Cu) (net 4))
 (segment (start 138.43 70.358) (end 138.43 68.02) (width 0.8128) (layer B.Cu) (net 4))
 (segment (start 135.8392 76.1192) (end 135.92 76.2) (width 0.8128) (layer B.Cu) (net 4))
 (segment (start 135.8392 72.6948) (end 135.8392 76.1192) (width 0.8128) (layer B.Cu) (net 4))
 (segment (start 130.735 65.226) (end 130.735 67.945) (width 0.508) (layer F.Cu) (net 5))
 (segment (start 132.08 63.881) (end 130.735 65.226) (width 0.508) (layer F.Cu) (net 5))
 (segment (start 138.565908 63.881) (end 132.08 63.881) (width 0.508) (layer F.Cu) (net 5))
 (segment (start 139.353308 64.6684) (end 138.565908 63.881) (width 0.508) (layer F.Cu) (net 5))
 (segment (start 140.7668 64.6684) (end 139.353308 64.6684) (width 0.508) (layer F.Cu) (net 5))
 (segment (start 140.004 74.524) (end 143.51 74.524) (width 1.27) (layer F.Cu) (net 6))
 (segment (start 138.505 73.025) (end 140.004 74.524) (width 1.27) (layer F.Cu) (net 6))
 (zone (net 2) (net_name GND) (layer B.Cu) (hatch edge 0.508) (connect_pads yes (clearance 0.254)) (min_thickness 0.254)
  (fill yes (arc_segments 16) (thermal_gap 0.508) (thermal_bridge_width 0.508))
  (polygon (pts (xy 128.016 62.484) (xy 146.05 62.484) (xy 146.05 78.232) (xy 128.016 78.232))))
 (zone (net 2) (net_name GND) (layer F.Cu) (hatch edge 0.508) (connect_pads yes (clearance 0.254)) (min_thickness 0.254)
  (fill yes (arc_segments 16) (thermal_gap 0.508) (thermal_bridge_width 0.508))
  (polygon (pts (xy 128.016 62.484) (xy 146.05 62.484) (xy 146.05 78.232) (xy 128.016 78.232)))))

